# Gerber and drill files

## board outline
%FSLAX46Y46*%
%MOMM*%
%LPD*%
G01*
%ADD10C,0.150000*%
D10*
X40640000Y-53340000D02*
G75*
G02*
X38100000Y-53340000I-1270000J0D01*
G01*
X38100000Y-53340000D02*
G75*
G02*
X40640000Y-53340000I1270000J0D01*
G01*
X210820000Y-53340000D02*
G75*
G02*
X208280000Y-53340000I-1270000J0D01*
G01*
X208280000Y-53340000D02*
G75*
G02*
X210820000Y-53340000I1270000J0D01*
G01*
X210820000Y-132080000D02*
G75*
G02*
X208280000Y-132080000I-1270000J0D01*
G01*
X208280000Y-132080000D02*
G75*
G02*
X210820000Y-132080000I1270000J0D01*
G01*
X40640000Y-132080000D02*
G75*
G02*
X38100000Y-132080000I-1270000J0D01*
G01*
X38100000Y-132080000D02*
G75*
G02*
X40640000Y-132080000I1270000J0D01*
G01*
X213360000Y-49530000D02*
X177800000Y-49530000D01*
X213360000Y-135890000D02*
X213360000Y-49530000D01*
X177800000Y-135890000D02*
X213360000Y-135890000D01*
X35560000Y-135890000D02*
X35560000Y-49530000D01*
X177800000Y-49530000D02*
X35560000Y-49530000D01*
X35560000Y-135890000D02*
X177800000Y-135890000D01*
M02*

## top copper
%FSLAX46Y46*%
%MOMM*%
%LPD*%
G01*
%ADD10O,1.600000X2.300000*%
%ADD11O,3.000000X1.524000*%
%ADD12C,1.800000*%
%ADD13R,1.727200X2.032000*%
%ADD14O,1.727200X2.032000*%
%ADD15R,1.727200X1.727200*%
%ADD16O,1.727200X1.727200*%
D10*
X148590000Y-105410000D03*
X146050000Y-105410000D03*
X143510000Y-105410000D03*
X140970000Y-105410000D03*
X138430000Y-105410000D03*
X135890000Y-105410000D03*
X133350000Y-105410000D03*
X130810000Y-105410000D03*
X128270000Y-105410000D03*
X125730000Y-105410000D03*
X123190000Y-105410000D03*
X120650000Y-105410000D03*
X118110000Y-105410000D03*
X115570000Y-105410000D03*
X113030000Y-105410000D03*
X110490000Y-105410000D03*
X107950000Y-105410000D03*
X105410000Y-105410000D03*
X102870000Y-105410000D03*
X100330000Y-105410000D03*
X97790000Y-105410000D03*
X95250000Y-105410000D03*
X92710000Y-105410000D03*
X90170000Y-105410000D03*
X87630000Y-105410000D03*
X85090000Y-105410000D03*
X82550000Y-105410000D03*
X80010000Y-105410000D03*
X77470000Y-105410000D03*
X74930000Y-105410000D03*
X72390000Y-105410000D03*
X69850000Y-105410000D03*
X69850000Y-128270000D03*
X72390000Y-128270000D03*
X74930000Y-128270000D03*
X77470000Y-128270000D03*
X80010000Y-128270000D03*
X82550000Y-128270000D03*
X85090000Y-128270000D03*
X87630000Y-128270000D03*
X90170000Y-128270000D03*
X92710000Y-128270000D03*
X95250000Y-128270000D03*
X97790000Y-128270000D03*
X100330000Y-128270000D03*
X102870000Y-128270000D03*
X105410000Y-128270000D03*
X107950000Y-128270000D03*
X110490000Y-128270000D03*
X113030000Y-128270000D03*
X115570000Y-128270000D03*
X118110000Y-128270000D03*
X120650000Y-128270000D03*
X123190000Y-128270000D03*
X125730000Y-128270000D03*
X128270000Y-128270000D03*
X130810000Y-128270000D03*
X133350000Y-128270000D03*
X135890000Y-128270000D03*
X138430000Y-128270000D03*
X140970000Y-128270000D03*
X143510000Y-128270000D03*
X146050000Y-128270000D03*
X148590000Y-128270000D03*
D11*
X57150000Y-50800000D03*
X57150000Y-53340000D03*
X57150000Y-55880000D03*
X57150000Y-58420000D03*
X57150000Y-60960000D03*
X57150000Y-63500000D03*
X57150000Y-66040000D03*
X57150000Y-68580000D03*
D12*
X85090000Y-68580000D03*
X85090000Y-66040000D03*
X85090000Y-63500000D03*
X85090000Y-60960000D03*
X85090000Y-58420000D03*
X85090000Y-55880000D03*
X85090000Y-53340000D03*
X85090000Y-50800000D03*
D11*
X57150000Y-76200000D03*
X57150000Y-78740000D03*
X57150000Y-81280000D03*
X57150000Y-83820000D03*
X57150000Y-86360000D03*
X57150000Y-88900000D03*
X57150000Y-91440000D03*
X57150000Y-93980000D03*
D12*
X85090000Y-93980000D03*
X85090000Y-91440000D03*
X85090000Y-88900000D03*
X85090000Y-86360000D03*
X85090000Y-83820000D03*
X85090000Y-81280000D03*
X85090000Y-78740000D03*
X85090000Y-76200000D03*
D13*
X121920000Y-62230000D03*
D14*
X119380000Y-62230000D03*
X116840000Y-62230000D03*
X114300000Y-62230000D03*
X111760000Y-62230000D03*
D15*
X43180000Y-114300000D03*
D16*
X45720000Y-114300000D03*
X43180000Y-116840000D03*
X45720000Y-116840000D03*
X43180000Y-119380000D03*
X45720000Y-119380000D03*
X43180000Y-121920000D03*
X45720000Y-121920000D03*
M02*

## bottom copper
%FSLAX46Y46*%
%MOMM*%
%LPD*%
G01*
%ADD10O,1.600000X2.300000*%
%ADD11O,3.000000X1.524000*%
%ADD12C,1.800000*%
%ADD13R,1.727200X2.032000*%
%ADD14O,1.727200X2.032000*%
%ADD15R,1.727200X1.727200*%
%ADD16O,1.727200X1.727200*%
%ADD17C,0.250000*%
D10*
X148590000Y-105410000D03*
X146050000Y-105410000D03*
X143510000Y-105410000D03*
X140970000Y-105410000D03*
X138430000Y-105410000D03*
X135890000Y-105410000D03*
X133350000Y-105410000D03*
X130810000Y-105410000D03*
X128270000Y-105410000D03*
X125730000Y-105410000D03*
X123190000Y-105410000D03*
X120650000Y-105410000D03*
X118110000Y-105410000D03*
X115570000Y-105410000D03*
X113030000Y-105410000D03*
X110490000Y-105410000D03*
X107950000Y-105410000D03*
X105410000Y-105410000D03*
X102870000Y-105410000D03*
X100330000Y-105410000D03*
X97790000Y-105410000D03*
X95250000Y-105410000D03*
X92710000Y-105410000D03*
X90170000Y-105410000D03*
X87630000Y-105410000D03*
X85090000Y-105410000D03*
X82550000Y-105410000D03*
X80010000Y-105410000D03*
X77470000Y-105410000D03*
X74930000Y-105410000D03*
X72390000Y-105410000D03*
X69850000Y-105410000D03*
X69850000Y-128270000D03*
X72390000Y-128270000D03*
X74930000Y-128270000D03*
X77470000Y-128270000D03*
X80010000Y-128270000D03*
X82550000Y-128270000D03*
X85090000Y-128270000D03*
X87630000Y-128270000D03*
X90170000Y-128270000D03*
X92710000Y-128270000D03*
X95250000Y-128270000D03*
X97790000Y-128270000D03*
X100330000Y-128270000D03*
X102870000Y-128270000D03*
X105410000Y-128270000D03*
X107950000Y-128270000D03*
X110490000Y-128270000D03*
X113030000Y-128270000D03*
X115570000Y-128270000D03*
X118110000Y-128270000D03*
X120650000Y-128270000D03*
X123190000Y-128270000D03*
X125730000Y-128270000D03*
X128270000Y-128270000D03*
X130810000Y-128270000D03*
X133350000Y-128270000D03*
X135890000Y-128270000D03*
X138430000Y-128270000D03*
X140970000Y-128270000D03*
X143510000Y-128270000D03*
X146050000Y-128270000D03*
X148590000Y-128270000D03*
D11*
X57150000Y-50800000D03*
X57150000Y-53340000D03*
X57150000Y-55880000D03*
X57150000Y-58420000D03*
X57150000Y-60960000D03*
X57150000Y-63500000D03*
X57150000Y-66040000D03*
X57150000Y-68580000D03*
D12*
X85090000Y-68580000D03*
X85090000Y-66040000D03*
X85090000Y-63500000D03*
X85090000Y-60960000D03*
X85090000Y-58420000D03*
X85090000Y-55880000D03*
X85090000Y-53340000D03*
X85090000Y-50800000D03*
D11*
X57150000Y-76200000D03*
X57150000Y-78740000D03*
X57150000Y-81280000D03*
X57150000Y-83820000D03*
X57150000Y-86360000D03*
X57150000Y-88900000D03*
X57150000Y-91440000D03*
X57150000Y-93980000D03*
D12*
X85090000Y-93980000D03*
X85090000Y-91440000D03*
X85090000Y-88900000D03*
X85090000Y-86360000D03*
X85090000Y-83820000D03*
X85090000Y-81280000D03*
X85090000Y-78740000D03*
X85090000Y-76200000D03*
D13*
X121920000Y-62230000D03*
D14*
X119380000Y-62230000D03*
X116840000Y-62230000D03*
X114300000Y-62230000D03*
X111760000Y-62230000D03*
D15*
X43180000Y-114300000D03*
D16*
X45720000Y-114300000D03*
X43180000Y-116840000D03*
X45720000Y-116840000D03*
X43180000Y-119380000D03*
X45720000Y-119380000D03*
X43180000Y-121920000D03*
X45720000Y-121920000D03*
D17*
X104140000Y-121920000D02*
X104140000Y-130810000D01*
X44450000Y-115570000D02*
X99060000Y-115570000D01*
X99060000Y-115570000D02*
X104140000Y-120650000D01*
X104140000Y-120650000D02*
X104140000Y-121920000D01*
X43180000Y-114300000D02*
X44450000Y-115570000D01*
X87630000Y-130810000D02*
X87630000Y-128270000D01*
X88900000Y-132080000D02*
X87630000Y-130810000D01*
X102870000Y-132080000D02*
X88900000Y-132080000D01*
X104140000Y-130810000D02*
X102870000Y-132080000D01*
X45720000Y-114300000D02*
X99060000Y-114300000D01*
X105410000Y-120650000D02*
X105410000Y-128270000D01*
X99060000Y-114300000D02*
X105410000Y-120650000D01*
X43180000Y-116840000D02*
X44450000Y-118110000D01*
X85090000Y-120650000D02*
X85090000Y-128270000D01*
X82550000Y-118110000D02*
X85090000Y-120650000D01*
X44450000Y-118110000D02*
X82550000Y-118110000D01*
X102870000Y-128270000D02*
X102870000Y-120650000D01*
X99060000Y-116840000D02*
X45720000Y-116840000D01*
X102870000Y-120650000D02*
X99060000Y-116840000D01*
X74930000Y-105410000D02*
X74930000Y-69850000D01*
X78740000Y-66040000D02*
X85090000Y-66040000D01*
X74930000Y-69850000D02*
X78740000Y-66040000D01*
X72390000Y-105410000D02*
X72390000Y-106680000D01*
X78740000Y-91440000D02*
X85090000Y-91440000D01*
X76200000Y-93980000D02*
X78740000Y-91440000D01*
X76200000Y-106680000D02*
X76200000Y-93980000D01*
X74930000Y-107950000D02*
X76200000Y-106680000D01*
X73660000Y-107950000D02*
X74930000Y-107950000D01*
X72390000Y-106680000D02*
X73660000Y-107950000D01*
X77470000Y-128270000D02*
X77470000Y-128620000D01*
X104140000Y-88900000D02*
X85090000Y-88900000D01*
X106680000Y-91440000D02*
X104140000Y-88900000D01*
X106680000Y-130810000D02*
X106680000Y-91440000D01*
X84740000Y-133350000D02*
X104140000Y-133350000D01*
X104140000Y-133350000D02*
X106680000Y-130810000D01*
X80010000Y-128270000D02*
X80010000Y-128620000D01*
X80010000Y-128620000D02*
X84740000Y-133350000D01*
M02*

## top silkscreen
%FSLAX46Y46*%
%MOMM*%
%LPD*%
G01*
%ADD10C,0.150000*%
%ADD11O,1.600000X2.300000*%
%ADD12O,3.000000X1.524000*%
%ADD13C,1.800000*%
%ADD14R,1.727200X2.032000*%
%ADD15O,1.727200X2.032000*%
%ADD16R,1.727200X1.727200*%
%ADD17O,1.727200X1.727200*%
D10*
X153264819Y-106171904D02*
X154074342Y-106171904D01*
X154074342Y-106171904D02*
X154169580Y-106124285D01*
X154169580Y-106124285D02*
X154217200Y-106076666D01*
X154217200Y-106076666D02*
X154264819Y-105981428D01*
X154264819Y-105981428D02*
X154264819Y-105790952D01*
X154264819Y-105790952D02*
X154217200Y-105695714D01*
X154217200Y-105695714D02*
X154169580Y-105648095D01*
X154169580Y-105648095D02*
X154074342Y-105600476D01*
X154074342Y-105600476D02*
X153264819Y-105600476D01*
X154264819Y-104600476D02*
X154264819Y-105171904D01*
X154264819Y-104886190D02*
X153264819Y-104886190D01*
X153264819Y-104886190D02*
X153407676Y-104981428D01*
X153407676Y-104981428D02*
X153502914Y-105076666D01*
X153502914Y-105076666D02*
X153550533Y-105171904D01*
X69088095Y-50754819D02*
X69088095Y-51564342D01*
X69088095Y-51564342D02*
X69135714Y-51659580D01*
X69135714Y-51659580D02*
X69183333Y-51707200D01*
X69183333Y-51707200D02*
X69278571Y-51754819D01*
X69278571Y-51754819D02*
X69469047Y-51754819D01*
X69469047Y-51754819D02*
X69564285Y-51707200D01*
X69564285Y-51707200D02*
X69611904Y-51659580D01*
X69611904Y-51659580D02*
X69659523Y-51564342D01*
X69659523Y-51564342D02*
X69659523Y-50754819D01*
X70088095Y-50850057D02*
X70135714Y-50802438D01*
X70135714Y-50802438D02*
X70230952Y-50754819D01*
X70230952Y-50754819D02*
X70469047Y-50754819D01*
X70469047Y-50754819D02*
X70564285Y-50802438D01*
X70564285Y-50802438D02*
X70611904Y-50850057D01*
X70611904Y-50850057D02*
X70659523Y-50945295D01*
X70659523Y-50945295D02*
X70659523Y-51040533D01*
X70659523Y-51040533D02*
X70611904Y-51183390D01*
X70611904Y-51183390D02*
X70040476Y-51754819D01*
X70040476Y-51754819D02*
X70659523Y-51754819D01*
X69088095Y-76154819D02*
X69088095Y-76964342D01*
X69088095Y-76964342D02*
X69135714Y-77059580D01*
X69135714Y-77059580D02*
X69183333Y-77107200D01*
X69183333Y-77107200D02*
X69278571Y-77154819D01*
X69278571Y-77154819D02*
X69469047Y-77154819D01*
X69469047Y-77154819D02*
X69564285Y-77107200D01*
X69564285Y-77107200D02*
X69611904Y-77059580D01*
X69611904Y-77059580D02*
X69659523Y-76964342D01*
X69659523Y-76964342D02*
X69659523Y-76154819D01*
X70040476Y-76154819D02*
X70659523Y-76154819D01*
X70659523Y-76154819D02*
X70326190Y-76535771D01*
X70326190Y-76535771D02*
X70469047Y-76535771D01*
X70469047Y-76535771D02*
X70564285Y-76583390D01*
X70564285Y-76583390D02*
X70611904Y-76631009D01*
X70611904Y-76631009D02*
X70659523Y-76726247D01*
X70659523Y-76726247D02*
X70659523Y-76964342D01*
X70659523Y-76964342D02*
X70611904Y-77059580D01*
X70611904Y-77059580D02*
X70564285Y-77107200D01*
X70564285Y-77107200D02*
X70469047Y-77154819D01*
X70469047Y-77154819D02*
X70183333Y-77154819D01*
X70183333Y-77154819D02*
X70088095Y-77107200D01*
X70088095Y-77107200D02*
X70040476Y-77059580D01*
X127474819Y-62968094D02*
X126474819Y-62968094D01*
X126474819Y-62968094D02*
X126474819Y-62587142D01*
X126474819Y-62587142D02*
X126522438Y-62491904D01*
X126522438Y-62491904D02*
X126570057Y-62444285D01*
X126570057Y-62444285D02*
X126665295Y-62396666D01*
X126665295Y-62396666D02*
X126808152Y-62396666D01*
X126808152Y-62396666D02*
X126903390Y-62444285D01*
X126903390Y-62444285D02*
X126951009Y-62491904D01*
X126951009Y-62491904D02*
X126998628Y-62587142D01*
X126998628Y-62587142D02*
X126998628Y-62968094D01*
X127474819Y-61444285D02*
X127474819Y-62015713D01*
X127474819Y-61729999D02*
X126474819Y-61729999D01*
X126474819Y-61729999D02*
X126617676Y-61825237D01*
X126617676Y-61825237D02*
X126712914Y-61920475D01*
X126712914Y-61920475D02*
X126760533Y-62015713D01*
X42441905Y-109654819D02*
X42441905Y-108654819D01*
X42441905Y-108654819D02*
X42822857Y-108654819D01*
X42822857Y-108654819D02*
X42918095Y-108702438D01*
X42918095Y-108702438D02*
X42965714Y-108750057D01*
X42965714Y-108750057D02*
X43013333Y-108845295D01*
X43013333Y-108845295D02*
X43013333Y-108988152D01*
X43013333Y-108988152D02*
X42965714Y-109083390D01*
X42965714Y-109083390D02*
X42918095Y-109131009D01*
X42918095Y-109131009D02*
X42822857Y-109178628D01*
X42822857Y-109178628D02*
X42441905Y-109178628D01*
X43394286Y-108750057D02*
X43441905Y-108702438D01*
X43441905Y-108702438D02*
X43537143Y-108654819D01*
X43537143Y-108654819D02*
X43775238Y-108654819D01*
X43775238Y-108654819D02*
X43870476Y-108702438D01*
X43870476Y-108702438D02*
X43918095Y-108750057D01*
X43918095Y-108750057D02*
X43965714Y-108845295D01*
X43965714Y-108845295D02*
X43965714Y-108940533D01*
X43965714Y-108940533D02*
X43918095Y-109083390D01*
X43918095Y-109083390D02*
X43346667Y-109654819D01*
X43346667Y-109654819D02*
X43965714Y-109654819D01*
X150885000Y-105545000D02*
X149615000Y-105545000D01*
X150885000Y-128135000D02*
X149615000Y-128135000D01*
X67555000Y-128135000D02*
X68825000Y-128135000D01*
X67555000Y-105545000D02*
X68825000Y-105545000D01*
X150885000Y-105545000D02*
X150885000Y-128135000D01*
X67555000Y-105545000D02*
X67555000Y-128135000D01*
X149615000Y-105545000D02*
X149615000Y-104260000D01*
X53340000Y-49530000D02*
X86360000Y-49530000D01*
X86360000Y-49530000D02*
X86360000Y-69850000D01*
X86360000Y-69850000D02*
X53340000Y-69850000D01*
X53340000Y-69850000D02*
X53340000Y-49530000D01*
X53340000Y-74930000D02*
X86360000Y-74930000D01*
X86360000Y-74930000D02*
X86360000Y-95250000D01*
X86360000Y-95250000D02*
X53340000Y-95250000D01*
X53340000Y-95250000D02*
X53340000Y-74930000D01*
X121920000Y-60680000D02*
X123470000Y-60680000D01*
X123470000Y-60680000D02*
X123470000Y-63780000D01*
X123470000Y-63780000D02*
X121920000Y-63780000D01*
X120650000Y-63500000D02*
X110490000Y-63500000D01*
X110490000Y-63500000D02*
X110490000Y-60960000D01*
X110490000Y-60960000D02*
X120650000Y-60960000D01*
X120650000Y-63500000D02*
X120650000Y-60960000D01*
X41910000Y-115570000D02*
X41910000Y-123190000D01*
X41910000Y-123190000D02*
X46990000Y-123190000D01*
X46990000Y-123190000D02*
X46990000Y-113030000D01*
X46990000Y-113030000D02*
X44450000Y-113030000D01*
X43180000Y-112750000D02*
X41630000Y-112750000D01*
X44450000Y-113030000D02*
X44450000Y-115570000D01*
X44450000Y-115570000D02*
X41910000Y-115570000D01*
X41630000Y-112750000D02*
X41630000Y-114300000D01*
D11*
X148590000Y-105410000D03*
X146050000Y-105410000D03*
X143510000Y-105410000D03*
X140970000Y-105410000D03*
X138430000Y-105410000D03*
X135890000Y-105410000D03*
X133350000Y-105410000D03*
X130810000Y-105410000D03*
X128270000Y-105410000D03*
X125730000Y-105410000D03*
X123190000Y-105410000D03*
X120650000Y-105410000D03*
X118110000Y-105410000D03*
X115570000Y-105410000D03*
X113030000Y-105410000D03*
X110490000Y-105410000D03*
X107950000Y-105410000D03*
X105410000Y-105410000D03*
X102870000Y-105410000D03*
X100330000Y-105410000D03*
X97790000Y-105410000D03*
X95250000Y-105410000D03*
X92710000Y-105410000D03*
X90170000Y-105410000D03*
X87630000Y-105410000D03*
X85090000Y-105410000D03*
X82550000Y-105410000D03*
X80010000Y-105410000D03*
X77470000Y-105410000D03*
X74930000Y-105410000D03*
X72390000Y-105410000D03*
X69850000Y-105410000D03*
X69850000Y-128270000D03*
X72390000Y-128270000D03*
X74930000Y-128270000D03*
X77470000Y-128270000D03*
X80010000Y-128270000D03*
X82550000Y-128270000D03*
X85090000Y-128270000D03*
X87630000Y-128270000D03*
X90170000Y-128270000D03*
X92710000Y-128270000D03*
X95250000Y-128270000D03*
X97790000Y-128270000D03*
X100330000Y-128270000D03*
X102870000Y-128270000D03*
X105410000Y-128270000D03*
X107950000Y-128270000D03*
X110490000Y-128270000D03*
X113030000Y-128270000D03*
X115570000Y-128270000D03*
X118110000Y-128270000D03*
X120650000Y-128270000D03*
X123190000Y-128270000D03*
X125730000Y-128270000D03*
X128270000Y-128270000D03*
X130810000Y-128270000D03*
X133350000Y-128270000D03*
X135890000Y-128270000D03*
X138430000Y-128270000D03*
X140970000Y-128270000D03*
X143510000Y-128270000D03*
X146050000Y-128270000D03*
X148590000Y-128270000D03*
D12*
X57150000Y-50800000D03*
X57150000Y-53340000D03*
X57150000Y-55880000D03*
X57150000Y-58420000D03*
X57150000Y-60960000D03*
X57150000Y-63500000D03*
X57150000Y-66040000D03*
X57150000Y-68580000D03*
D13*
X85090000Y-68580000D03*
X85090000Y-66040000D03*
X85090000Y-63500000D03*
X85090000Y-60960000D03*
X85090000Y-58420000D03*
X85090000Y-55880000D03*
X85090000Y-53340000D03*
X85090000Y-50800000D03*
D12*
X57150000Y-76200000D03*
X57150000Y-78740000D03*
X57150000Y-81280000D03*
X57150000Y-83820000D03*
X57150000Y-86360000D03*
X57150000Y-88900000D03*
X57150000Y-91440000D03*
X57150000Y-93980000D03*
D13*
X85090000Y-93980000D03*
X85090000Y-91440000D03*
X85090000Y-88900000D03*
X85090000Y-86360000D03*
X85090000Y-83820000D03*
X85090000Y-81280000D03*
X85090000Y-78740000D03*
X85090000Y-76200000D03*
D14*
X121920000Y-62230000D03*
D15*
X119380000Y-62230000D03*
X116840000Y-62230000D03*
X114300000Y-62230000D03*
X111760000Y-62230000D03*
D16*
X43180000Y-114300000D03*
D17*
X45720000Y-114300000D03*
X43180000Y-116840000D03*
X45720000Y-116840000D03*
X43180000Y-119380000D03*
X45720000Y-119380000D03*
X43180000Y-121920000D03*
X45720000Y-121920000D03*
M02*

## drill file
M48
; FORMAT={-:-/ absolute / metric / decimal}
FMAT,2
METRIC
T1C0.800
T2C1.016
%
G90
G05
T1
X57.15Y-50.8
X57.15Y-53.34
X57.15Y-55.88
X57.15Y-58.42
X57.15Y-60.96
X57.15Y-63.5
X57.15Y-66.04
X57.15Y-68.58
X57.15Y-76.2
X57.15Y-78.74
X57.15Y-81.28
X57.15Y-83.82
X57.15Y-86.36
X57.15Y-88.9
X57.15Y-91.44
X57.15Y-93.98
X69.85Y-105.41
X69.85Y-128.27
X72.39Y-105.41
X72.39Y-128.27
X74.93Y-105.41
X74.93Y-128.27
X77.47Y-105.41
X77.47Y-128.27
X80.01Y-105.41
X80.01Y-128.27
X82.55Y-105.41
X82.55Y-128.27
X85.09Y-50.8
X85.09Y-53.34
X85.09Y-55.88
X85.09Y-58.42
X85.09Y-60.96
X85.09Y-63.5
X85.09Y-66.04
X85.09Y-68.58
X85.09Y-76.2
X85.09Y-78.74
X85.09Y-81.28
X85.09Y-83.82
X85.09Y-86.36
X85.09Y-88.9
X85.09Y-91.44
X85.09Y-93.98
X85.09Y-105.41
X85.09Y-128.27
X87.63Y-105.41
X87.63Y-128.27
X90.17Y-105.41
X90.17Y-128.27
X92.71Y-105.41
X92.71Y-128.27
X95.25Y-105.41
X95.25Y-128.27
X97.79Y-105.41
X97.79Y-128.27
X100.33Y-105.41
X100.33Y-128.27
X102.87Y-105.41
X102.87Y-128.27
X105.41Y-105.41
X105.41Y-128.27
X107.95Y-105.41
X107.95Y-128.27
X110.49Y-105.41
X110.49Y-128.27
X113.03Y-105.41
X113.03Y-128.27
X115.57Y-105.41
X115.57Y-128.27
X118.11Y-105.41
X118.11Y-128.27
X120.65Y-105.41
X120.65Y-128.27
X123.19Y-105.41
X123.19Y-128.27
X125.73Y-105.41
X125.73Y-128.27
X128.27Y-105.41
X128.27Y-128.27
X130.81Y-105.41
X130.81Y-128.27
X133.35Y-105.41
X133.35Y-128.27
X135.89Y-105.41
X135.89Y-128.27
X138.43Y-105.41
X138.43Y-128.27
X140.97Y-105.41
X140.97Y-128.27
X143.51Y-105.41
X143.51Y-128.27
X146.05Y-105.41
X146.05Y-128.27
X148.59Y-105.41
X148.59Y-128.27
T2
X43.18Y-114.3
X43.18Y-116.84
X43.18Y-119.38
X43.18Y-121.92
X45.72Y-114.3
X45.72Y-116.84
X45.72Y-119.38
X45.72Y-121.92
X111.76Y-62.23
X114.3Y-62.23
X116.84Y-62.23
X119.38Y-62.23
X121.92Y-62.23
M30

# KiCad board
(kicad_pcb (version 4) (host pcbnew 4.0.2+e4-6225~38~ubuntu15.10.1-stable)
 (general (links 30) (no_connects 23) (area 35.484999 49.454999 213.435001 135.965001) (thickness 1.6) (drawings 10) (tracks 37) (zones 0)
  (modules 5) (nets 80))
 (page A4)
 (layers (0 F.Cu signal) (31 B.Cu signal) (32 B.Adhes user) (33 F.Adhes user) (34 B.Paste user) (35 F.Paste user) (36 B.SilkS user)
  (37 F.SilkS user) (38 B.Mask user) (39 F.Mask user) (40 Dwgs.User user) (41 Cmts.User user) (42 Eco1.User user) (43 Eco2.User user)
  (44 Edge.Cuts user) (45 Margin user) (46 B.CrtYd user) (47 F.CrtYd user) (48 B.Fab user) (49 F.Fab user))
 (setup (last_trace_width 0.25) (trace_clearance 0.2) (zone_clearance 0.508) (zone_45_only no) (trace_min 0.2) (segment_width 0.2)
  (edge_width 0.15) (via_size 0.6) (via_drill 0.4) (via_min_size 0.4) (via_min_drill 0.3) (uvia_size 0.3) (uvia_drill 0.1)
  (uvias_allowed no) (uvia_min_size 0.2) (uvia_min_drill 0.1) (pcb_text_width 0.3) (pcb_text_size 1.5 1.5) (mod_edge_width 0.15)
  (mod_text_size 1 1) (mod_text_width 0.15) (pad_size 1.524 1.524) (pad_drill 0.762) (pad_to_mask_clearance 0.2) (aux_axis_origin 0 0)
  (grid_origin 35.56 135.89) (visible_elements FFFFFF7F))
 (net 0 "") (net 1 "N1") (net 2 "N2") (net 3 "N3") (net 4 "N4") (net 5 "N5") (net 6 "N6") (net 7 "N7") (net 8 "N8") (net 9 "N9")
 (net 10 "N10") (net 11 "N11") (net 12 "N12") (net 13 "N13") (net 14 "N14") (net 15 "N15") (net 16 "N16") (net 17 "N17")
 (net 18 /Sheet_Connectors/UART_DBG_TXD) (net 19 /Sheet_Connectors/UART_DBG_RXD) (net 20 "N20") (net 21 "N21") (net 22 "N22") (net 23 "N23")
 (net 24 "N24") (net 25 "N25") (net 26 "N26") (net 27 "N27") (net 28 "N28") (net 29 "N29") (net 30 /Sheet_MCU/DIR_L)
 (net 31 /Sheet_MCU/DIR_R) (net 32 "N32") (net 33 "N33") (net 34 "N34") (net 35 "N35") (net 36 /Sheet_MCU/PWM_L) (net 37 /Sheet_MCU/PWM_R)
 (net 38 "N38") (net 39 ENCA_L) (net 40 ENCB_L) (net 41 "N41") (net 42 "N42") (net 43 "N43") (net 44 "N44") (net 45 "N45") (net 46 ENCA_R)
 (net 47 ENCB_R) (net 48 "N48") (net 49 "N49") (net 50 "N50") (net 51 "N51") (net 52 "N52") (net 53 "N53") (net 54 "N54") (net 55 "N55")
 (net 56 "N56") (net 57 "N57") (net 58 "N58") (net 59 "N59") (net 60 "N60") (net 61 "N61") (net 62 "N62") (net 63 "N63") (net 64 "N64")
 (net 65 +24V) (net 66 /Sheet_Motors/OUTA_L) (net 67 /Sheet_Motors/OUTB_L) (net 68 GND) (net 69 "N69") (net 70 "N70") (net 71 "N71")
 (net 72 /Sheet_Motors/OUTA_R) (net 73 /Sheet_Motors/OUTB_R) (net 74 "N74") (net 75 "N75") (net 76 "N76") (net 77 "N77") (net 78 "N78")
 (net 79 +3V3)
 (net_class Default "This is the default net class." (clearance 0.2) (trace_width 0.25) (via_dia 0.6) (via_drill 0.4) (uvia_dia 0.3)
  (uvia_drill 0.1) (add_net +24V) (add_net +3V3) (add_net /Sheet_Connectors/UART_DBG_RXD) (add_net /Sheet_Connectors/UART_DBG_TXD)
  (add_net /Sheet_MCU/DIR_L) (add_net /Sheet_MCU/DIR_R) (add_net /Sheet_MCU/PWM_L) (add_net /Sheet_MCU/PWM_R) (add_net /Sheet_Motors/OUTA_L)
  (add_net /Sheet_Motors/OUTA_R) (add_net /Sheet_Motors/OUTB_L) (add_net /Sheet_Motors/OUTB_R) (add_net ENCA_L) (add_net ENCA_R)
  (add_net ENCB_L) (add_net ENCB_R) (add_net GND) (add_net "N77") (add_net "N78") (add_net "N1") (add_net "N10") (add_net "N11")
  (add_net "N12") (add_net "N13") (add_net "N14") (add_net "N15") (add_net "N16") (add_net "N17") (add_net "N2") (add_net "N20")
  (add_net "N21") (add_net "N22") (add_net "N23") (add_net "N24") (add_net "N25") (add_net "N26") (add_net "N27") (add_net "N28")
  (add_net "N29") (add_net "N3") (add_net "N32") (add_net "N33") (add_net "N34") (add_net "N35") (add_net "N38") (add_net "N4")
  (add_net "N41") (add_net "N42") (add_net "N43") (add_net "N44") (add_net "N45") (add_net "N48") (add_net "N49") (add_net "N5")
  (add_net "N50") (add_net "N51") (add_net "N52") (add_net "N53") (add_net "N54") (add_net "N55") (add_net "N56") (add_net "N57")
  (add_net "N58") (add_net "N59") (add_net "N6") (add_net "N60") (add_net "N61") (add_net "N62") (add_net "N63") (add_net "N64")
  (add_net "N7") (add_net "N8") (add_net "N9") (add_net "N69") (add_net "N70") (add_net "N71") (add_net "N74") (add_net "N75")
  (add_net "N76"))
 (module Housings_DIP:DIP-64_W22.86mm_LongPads (layer F.Cu) (at 148.59 105.41 270)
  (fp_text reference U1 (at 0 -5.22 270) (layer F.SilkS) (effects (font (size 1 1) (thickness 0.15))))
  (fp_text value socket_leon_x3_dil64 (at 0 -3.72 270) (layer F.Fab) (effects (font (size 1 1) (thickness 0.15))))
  (fp_line (start 0.135 -2.295) (end 0.135 -1.025) (layer F.SilkS) (width 0.15))
  (fp_line (start 22.725 -2.295) (end 22.725 -1.025) (layer F.SilkS) (width 0.15))
  (fp_line (start 22.725 81.035) (end 22.725 79.765) (layer F.SilkS) (width 0.15))
  (fp_line (start 0.135 81.035) (end 0.135 79.765) (layer F.SilkS) (width 0.15))
  (fp_line (start 0.135 -2.295) (end 22.725 -2.295) (layer F.SilkS) (width 0.15))
  (fp_line (start 0.135 81.035) (end 22.725 81.035) (layer F.SilkS) (width 0.15))
  (fp_line (start 0.135 -1.025) (end -1.15 -1.025) (layer F.SilkS) (width 0.15))
  (pad 1 thru_hole oval (at 0 0 270) (size 2.3 1.6) (drill 0.8) (layers *.Cu *.Mask F.SilkS) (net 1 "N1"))
  (pad 2 thru_hole oval (at 0 2.54 270) (size 2.3 1.6) (drill 0.8) (layers *.Cu *.Mask F.SilkS) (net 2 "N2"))
  (pad 3 thru_hole oval (at 0 5.08 270) (size 2.3 1.6) (drill 0.8) (layers *.Cu *.Mask F.SilkS) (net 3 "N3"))
  (pad 4 thru_hole oval (at 0 7.62 270) (size 2.3 1.6) (drill 0.8) (layers *.Cu *.Mask F.SilkS) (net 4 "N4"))
  (pad 5 thru_hole oval (at 0 10.16 270) (size 2.3 1.6) (drill 0.8) (layers *.Cu *.Mask F.SilkS) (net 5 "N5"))
  (pad 6 thru_hole oval (at 0 12.7 270) (size 2.3 1.6) (drill 0.8) (layers *.Cu *.Mask F.SilkS) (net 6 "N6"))
  (pad 7 thru_hole oval (at 0 15.24 270) (size 2.3 1.6) (drill 0.8) (layers *.Cu *.Mask F.SilkS) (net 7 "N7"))
  (pad 8 thru_hole oval (at 0 17.78 270) (size 2.3 1.6) (drill 0.8) (layers *.Cu *.Mask F.SilkS) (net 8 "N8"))
  (pad 9 thru_hole oval (at 0 20.32 270) (size 2.3 1.6) (drill 0.8) (layers *.Cu *.Mask F.SilkS) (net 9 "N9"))
  (pad 10 thru_hole oval (at 0 22.86 270) (size 2.3 1.6) (drill 0.8) (layers *.Cu *.Mask F.SilkS) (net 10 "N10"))
  (pad 11 thru_hole oval (at 0 25.4 270) (size 2.3 1.6) (drill 0.8) (layers *.Cu *.Mask F.SilkS) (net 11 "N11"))
  (pad 12 thru_hole oval (at 0 27.94 270) (size 2.3 1.6) (drill 0.8) (layers *.Cu *.Mask F.SilkS) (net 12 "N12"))
  (pad 13 thru_hole oval (at 0 30.48 270) (size 2.3 1.6) (drill 0.8) (layers *.Cu *.Mask F.SilkS) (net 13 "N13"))
  (pad 14 thru_hole oval (at 0 33.02 270) (size 2.3 1.6) (drill 0.8) (layers *.Cu *.Mask F.SilkS) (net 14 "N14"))
  (pad 15 thru_hole oval (at 0 35.56 270) (size 2.3 1.6) (drill 0.8) (layers *.Cu *.Mask F.SilkS) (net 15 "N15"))
  (pad 16 thru_hole oval (at 0 38.1 270) (size 2.3 1.6) (drill 0.8) (layers *.Cu *.Mask F.SilkS) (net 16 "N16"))
  (pad 17 thru_hole oval (at 0 40.64 270) (size 2.3 1.6) (drill 0.8) (layers *.Cu *.Mask F.SilkS) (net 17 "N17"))
  (pad 18 thru_hole oval (at 0 43.18 270) (size 2.3 1.6) (drill 0.8) (layers *.Cu *.Mask F.SilkS) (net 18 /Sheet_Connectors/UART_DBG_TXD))
  (pad 19 thru_hole oval (at 0 45.72 270) (size 2.3 1.6) (drill 0.8) (layers *.Cu *.Mask F.SilkS) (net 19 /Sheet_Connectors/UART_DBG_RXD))
  (pad 20 thru_hole oval (at 0 48.26 270) (size 2.3 1.6) (drill 0.8) (layers *.Cu *.Mask F.SilkS) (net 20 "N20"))
  (pad 21 thru_hole oval (at 0 50.8 270) (size 2.3 1.6) (drill 0.8) (layers *.Cu *.Mask F.SilkS) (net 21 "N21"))
  (pad 22 thru_hole oval (at 0 53.34 270) (size 2.3 1.6) (drill 0.8) (layers *.Cu *.Mask F.SilkS) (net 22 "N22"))
  (pad 23 thru_hole oval (at 0 55.88 270) (size 2.3 1.6) (drill 0.8) (layers *.Cu *.Mask F.SilkS) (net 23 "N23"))
  (pad 24 thru_hole oval (at 0 58.42 270) (size 2.3 1.6) (drill 0.8) (layers *.Cu *.Mask F.SilkS) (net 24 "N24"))
  (pad 25 thru_hole oval (at 0 60.96 270) (size 2.3 1.6) (drill 0.8) (layers *.Cu *.Mask F.SilkS) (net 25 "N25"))
  (pad 26 thru_hole oval (at 0 63.5 270) (size 2.3 1.6) (drill 0.8) (layers *.Cu *.Mask F.SilkS) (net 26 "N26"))
  (pad 27 thru_hole oval (at 0 66.04 270) (size 2.3 1.6) (drill 0.8) (layers *.Cu *.Mask F.SilkS) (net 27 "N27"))
  (pad 28 thru_hole oval (at 0 68.58 270) (size 2.3 1.6) (drill 0.8) (layers *.Cu *.Mask F.SilkS) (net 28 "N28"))
  (pad 29 thru_hole oval (at 0 71.12 270) (size 2.3 1.6) (drill 0.8) (layers *.Cu *.Mask F.SilkS) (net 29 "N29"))
  (pad 30 thru_hole oval (at 0 73.66 270) (size 2.3 1.6) (drill 0.8) (layers *.Cu *.Mask F.SilkS) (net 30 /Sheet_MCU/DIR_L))
  (pad 31 thru_hole oval (at 0 76.2 270) (size 2.3 1.6) (drill 0.8) (layers *.Cu *.Mask F.SilkS) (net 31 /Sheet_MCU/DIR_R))
  (pad 32 thru_hole oval (at 0 78.74 270) (size 2.3 1.6) (drill 0.8) (layers *.Cu *.Mask F.SilkS) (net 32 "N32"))
  (pad 33 thru_hole oval (at 22.86 78.74 270) (size 2.3 1.6) (drill 0.8) (layers *.Cu *.Mask F.SilkS) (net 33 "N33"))
  (pad 34 thru_hole oval (at 22.86 76.2 270) (size 2.3 1.6) (drill 0.8) (layers *.Cu *.Mask F.SilkS) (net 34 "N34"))
  (pad 35 thru_hole oval (at 22.86 73.66 270) (size 2.3 1.6) (drill 0.8) (layers *.Cu *.Mask F.SilkS) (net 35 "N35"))
  (pad 36 thru_hole oval (at 22.86 71.12 270) (size 2.3 1.6) (drill 0.8) (layers *.Cu *.Mask F.SilkS) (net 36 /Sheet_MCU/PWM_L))
  (pad 37 thru_hole oval (at 22.86 68.58 270) (size 2.3 1.6) (drill 0.8) (layers *.Cu *.Mask F.SilkS) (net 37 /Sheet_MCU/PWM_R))
  (pad 38 thru_hole oval (at 22.86 66.04 270) (size 2.3 1.6) (drill 0.8) (layers *.Cu *.Mask F.SilkS) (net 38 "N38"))
  (pad 39 thru_hole oval (at 22.86 63.5 270) (size 2.3 1.6) (drill 0.8) (layers *.Cu *.Mask F.SilkS) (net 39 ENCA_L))
  (pad 40 thru_hole oval (at 22.86 60.96 270) (size 2.3 1.6) (drill 0.8) (layers *.Cu *.Mask F.SilkS) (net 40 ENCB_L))
  (pad 41 thru_hole oval (at 22.86 58.42 270) (size 2.3 1.6) (drill 0.8) (layers *.Cu *.Mask F.SilkS) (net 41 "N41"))
  (pad 42 thru_hole oval (at 22.86 55.88 270) (size 2.3 1.6) (drill 0.8) (layers *.Cu *.Mask F.SilkS) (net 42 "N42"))
  (pad 43 thru_hole oval (at 22.86 53.34 270) (size 2.3 1.6) (drill 0.8) (layers *.Cu *.Mask F.SilkS) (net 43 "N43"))
  (pad 44 thru_hole oval (at 22.86 50.8 270) (size 2.3 1.6) (drill 0.8) (layers *.Cu *.Mask F.SilkS) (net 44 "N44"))
  (pad 45 thru_hole oval (at 22.86 48.26 270) (size 2.3 1.6) (drill 0.8) (layers *.Cu *.Mask F.SilkS) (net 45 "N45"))
  (pad 46 thru_hole oval (at 22.86 45.72 270) (size 2.3 1.6) (drill 0.8) (layers *.Cu *.Mask F.SilkS) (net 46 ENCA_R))
  (pad 47 thru_hole oval (at 22.86 43.18 270) (size 2.3 1.6) (drill 0.8) (layers *.Cu *.Mask F.SilkS) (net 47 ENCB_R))
  (pad 48 thru_hole oval (at 22.86 40.64 270) (size 2.3 1.6) (drill 0.8) (layers *.Cu *.Mask F.SilkS) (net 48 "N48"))
  (pad 49 thru_hole oval (at 22.86 38.1 270) (size 2.3 1.6) (drill 0.8) (layers *.Cu *.Mask F.SilkS) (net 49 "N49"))
  (pad 50 thru_hole oval (at 22.86 35.56 270) (size 2.3 1.6) (drill 0.8) (layers *.Cu *.Mask F.SilkS) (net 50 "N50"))
  (pad 51 thru_hole oval (at 22.86 33.02 270) (size 2.3 1.6) (drill 0.8) (layers *.Cu *.Mask F.SilkS) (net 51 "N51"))
  (pad 52 thru_hole oval (at 22.86 30.48 270) (size 2.3 1.6) (drill 0.8) (layers *.Cu *.Mask F.SilkS) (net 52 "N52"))
  (pad 53 thru_hole oval (at 22.86 27.94 270) (size 2.3 1.6) (drill 0.8) (layers *.Cu *.Mask F.SilkS) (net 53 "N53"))
  (pad 54 thru_hole oval (at 22.86 25.4 270) (size 2.3 1.6) (drill 0.8) (layers *.Cu *.Mask F.SilkS) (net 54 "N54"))
  (pad 55 thru_hole oval (at 22.86 22.86 270) (size 2.3 1.6) (drill 0.8) (layers *.Cu *.Mask F.SilkS) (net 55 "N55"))
  (pad 56 thru_hole oval (at 22.86 20.32 270) (size 2.3 1.6) (drill 0.8) (layers *.Cu *.Mask F.SilkS) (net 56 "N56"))
  (pad 57 thru_hole oval (at 22.86 17.78 270) (size 2.3 1.6) (drill 0.8) (layers *.Cu *.Mask F.SilkS) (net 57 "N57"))
  (pad 58 thru_hole oval (at 22.86 15.24 270) (size 2.3 1.6) (drill 0.8) (layers *.Cu *.Mask F.SilkS) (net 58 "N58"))
  (pad 59 thru_hole oval (at 22.86 12.7 270) (size 2.3 1.6) (drill 0.8) (layers *.Cu *.Mask F.SilkS) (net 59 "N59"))
  (pad 60 thru_hole oval (at 22.86 10.16 270) (size 2.3 1.6) (drill 0.8) (layers *.Cu *.Mask F.SilkS) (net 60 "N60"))
  (pad 61 thru_hole oval (at 22.86 7.62 270) (size 2.3 1.6) (drill 0.8) (layers *.Cu *.Mask F.SilkS) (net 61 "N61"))
  (pad 62 thru_hole oval (at 22.86 5.08 270) (size 2.3 1.6) (drill 0.8) (layers *.Cu *.Mask F.SilkS) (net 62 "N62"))
  (pad 63 thru_hole oval (at 22.86 2.54 270) (size 2.3 1.6) (drill 0.8) (layers *.Cu *.Mask F.SilkS) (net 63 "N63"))
  (pad 64 thru_hole oval (at 22.86 0 270) (size 2.3 1.6) (drill 0.8) (layers *.Cu *.Mask F.SilkS) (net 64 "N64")))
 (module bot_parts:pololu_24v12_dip (layer F.Cu) (at 69.85 59.69)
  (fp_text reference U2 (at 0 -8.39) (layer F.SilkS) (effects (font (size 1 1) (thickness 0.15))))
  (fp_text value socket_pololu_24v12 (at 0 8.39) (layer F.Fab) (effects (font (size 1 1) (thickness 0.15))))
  (fp_line (start -16.51 -10.16) (end 16.51 -10.16) (layer F.SilkS) (width 0.15))
  (fp_line (start 16.51 -10.16) (end 16.51 10.16) (layer F.SilkS) (width 0.15))
  (fp_line (start 16.51 10.16) (end -16.51 10.16) (layer F.SilkS) (width 0.15))
  (fp_line (start -16.51 10.16) (end -16.51 -10.16) (layer F.SilkS) (width 0.15))
  (pad 1 thru_hole oval (at -12.7 -8.89) (size 3 1.524) (drill 0.8) (layers *.Cu *.Mask F.SilkS) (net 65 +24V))
  (pad 2 thru_hole oval (at -12.7 -6.35) (size 3 1.524) (drill 0.8) (layers *.Cu *.Mask F.SilkS) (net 65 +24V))
  (pad 3 thru_hole oval (at -12.7 -3.81) (size 3 1.524) (drill 0.8) (layers *.Cu *.Mask F.SilkS) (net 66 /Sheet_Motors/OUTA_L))
  (pad 4 thru_hole oval (at -12.7 -1.27) (size 3 1.524) (drill 0.8) (layers *.Cu *.Mask F.SilkS) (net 66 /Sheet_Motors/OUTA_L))
  (pad 5 thru_hole oval (at -12.7 1.27) (size 3 1.524) (drill 0.8) (layers *.Cu *.Mask F.SilkS) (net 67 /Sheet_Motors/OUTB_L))
  (pad 6 thru_hole oval (at -12.7 3.81) (size 3 1.524) (drill 0.8) (layers *.Cu *.Mask F.SilkS) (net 67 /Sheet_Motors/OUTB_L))
  (pad 7 thru_hole oval (at -12.7 6.35) (size 3 1.524) (drill 0.8) (layers *.Cu *.Mask F.SilkS) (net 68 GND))
  (pad 8 thru_hole oval (at -12.7 8.89) (size 3 1.524) (drill 0.8) (layers *.Cu *.Mask F.SilkS) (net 68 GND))
  (pad 9 thru_hole circle (at 15.24 8.89) (size 1.8 1.8) (drill 0.8) (layers *.Cu *.Mask F.SilkS) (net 68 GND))
  (pad 10 thru_hole circle (at 15.24 6.35) (size 1.8 1.8) (drill 0.8) (layers *.Cu *.Mask F.SilkS) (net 30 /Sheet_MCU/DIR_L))
  (pad 11 thru_hole circle (at 15.24 3.81) (size 1.8 1.8) (drill 0.8) (layers *.Cu *.Mask F.SilkS) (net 36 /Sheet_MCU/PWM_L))
  (pad 12 thru_hole circle (at 15.24 1.27) (size 1.8 1.8) (drill 0.8) (layers *.Cu *.Mask F.SilkS) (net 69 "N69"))
  (pad 13 thru_hole circle (at 15.24 -1.27) (size 1.8 1.8) (drill 0.8) (layers *.Cu *.Mask F.SilkS) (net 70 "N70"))
  (pad 14 thru_hole circle (at 15.24 -3.81) (size 1.8 1.8) (drill 0.8) (layers *.Cu *.Mask F.SilkS) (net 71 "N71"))
  (pad 15 thru_hole circle (at 15.24 -6.35) (size 1.8 1.8) (drill 0.8) (layers *.Cu *.Mask F.SilkS) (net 65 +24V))
  (pad 16 thru_hole circle (at 15.24 -8.89) (size 1.8 1.8) (drill 0.8) (layers *.Cu *.Mask F.SilkS) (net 65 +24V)))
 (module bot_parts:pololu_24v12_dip (layer F.Cu) (at 69.85 85.09)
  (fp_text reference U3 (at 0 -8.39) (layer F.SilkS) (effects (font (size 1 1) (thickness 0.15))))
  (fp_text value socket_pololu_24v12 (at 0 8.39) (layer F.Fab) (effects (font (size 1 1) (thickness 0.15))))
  (fp_line (start -16.51 -10.16) (end 16.51 -10.16) (layer F.SilkS) (width 0.15))
  (fp_line (start 16.51 -10.16) (end 16.51 10.16) (layer F.SilkS) (width 0.15))
  (fp_line (start 16.51 10.16) (end -16.51 10.16) (layer F.SilkS) (width 0.15))
  (fp_line (start -16.51 10.16) (end -16.51 -10.16) (layer F.SilkS) (width 0.15))
  (pad 1 thru_hole oval (at -12.7 -8.89) (size 3 1.524) (drill 0.8) (layers *.Cu *.Mask F.SilkS) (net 65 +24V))
  (pad 2 thru_hole oval (at -12.7 -6.35) (size 3 1.524) (drill 0.8) (layers *.Cu *.Mask F.SilkS) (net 65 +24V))
  (pad 3 thru_hole oval (at -12.7 -3.81) (size 3 1.524) (drill 0.8) (layers *.Cu *.Mask F.SilkS) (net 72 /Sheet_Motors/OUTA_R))
  (pad 4 thru_hole oval (at -12.7 -1.27) (size 3 1.524) (drill 0.8) (layers *.Cu *.Mask F.SilkS) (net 72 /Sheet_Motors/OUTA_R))
  (pad 5 thru_hole oval (at -12.7 1.27) (size 3 1.524) (drill 0.8) (layers *.Cu *.Mask F.SilkS) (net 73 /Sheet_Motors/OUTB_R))
  (pad 6 thru_hole oval (at -12.7 3.81) (size 3 1.524) (drill 0.8) (layers *.Cu *.Mask F.SilkS) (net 73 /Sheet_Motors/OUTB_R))
  (pad 7 thru_hole oval (at -12.7 6.35) (size 3 1.524) (drill 0.8) (layers *.Cu *.Mask F.SilkS) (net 68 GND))
  (pad 8 thru_hole oval (at -12.7 8.89) (size 3 1.524) (drill 0.8) (layers *.Cu *.Mask F.SilkS) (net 68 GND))
  (pad 9 thru_hole circle (at 15.24 8.89) (size 1.8 1.8) (drill 0.8) (layers *.Cu *.Mask F.SilkS) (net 68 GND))
  (pad 10 thru_hole circle (at 15.24 6.35) (size 1.8 1.8) (drill 0.8) (layers *.Cu *.Mask F.SilkS) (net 31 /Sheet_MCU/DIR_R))
  (pad 11 thru_hole circle (at 15.24 3.81) (size 1.8 1.8) (drill 0.8) (layers *.Cu *.Mask F.SilkS) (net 37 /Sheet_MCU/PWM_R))
  (pad 12 thru_hole circle (at 15.24 1.27) (size 1.8 1.8) (drill 0.8) (layers *.Cu *.Mask F.SilkS) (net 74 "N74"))
  (pad 13 thru_hole circle (at 15.24 -1.27) (size 1.8 1.8) (drill 0.8) (layers *.Cu *.Mask F.SilkS) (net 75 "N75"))
  (pad 14 thru_hole circle (at 15.24 -3.81) (size 1.8 1.8) (drill 0.8) (layers *.Cu *.Mask F.SilkS) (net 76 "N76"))
  (pad 15 thru_hole circle (at 15.24 -6.35) (size 1.8 1.8) (drill 0.8) (layers *.Cu *.Mask F.SilkS) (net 65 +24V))
  (pad 16 thru_hole circle (at 15.24 -8.89) (size 1.8 1.8) (drill 0.8) (layers *.Cu *.Mask F.SilkS) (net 65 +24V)))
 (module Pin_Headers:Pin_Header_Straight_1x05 (layer F.Cu) (at 121.92 62.23 270)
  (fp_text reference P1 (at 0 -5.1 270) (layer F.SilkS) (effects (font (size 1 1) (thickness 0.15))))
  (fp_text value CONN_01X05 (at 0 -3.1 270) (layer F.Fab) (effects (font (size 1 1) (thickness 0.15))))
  (fp_line (start -1.55 0) (end -1.55 -1.55) (layer F.SilkS) (width 0.15))
  (fp_line (start -1.55 -1.55) (end 1.55 -1.55) (layer F.SilkS) (width 0.15))
  (fp_line (start 1.55 -1.55) (end 1.55 0) (layer F.SilkS) (width 0.15))
  (fp_line (start 1.27 1.27) (end 1.27 11.43) (layer F.SilkS) (width 0.15))
  (fp_line (start 1.27 11.43) (end -1.27 11.43) (layer F.SilkS) (width 0.15))
  (fp_line (start -1.27 11.43) (end -1.27 1.27) (layer F.SilkS) (width 0.15))
  (fp_line (start 1.27 1.27) (end -1.27 1.27) (layer F.SilkS) (width 0.15))
  (pad 1 thru_hole rect (at 0 0 270) (size 2.032 1.7272) (drill 1.016) (layers *.Cu *.Mask F.SilkS) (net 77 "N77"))
  (pad 2 thru_hole oval (at 0 2.54 270) (size 2.032 1.7272) (drill 1.016) (layers *.Cu *.Mask F.SilkS)
   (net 18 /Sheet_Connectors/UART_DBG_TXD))
  (pad 3 thru_hole oval (at 0 5.08 270) (size 2.032 1.7272) (drill 1.016) (layers *.Cu *.Mask F.SilkS)
   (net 19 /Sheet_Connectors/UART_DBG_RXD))
  (pad 4 thru_hole oval (at 0 7.62 270) (size 2.032 1.7272) (drill 1.016) (layers *.Cu *.Mask F.SilkS) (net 68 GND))
  (pad 5 thru_hole oval (at 0 10.16 270) (size 2.032 1.7272) (drill 1.016) (layers *.Cu *.Mask F.SilkS) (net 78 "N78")))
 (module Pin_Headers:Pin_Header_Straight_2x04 (layer F.Cu) (at 43.18 114.3)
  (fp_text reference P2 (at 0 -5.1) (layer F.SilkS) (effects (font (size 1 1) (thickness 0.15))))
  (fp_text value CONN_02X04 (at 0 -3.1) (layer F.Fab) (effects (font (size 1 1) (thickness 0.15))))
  (fp_line (start -1.27 1.27) (end -1.27 8.89) (layer F.SilkS) (width 0.15))
  (fp_line (start -1.27 8.89) (end 3.81 8.89) (layer F.SilkS) (width 0.15))
  (fp_line (start 3.81 8.89) (end 3.81 -1.27) (layer F.SilkS) (width 0.15))
  (fp_line (start 3.81 -1.27) (end 1.27 -1.27) (layer F.SilkS) (width 0.15))
  (fp_line (start 0 -1.55) (end -1.55 -1.55) (layer F.SilkS) (width 0.15))
  (fp_line (start 1.27 -1.27) (end 1.27 1.27) (layer F.SilkS) (width 0.15))
  (fp_line (start 1.27 1.27) (end -1.27 1.27) (layer F.SilkS) (width 0.15))
  (fp_line (start -1.55 -1.55) (end -1.55 0) (layer F.SilkS) (width 0.15))
  (pad 1 thru_hole rect (at 0 0) (size 1.7272 1.7272) (drill 1.016) (layers *.Cu *.Mask F.SilkS) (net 40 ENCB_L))
  (pad 2 thru_hole oval (at 2.54 0) (size 1.7272 1.7272) (drill 1.016) (layers *.Cu *.Mask F.SilkS) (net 47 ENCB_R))
  (pad 3 thru_hole oval (at 0 2.54) (size 1.7272 1.7272) (drill 1.016) (layers *.Cu *.Mask F.SilkS) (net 39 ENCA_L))
  (pad 4 thru_hole oval (at 2.54 2.54) (size 1.7272 1.7272) (drill 1.016) (layers *.Cu *.Mask F.SilkS) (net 46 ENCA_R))
  (pad 5 thru_hole oval (at 0 5.08) (size 1.7272 1.7272) (drill 1.016) (layers *.Cu *.Mask F.SilkS) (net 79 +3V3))
  (pad 6 thru_hole oval (at 2.54 5.08) (size 1.7272 1.7272) (drill 1.016) (layers *.Cu *.Mask F.SilkS) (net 79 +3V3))
  (pad 7 thru_hole oval (at 0 7.62) (size 1.7272 1.7272) (drill 1.016) (layers *.Cu *.Mask F.SilkS) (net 68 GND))
  (pad 8 thru_hole oval (at 2.54 7.62) (size 1.7272 1.7272) (drill 1.016) (layers *.Cu *.Mask F.SilkS) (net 68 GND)))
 (gr_circle (center 39.37 53.34) (end 40.64 53.34) (layer Edge.Cuts) (width 0.15))
 (gr_circle (center 209.55 53.34) (end 209.55 52.07) (layer Edge.Cuts) (width 0.15))
 (gr_circle (center 209.55 132.08) (end 210.82 132.08) (layer Edge.Cuts) (width 0.15))
 (gr_circle (center 39.37 132.08) (end 40.64 132.08) (layer Edge.Cuts) (width 0.15))
 (gr_line (start 213.36 49.53) (end 177.8 49.53) (angle 90) (layer Edge.Cuts) (width 0.15))
 (gr_line (start 213.36 135.89) (end 213.36 49.53) (angle 90) (layer Edge.Cuts) (width 0.15))
 (gr_line (start 177.8 135.89) (end 213.36 135.89) (angle 90) (layer Edge.Cuts) (width 0.15))
 (gr_line (start 35.56 135.89) (end 35.56 49.53) (angle 90) (layer Edge.Cuts) (width 0.15))
 (gr_line (start 177.8 49.53) (end 35.56 49.53) (angle 90) (layer Edge.Cuts) (width 0.15))
 (gr_line (start 35.56 135.89) (end 177.8 135.89) (angle 90) (layer Edge.Cuts) (width 0.15))
 (segment (start 104.14 121.92) (end 104.14 130.81) (width 0.25) (layer B.Cu) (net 40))
 (segment (start 44.45 115.57) (end 99.06 115.57) (width 0.25) (layer B.Cu) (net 40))
 (segment (start 99.06 115.57) (end 104.14 120.65) (width 0.25) (layer B.Cu) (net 40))
 (segment (start 104.14 120.65) (end 104.14 121.92) (width 0.25) (layer B.Cu) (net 40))
 (segment (start 43.18 114.3) (end 44.45 115.57) (width 0.25) (layer B.Cu) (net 40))
 (segment (start 87.63 130.81) (end 87.63 128.27) (width 0.25) (layer B.Cu) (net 40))
 (segment (start 88.9 132.08) (end 87.63 130.81) (width 0.25) (layer B.Cu) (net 40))
 (segment (start 102.87 132.08) (end 88.9 132.08) (width 0.25) (layer B.Cu) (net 40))
 (segment (start 104.14 130.81) (end 102.87 132.08) (width 0.25) (layer B.Cu) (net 40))
 (segment (start 45.72 114.3) (end 99.06 114.3) (width 0.25) (layer B.Cu) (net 47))
 (segment (start 105.41 120.65) (end 105.41 128.27) (width 0.25) (layer B.Cu) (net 47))
 (segment (start 99.06 114.3) (end 105.41 120.65) (width 0.25) (layer B.Cu) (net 47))
 (segment (start 43.18 116.84) (end 44.45 118.11) (width 0.25) (layer B.Cu) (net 39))
 (segment (start 85.09 120.65) (end 85.09 128.27) (width 0.25) (layer B.Cu) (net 39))
 (segment (start 82.55 118.11) (end 85.09 120.65) (width 0.25) (layer B.Cu) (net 39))
 (segment (start 44.45 118.11) (end 82.55 118.11) (width 0.25) (layer B.Cu) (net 39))
 (segment (start 102.87 128.27) (end 102.87 120.65) (width 0.25) (layer B.Cu) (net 46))
 (segment (start 99.06 116.84) (end 45.72 116.84) (width 0.25) (layer B.Cu) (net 46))
 (segment (start 102.87 120.65) (end 99.06 116.84) (width 0.25) (layer B.Cu) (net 46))
 (segment (start 74.93 105.41) (end 74.93 69.85) (width 0.25) (layer B.Cu) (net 30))
 (segment (start 78.74 66.04) (end 85.09 66.04) (width 0.25) (layer B.Cu) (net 30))
 (segment (start 74.93 69.85) (end 78.74 66.04) (width 0.25) (layer B.Cu) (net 30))
 (segment (start 72.39 105.41) (end 72.39 106.68) (width 0.25) (layer B.Cu) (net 31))
 (segment (start 78.74 91.44) (end 85.09 91.44) (width 0.25) (layer B.Cu) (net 31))
 (segment (start 76.2 93.98) (end 78.74 91.44) (width 0.25) (layer B.Cu) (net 31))
 (segment (start 76.2 106.68) (end 76.2 93.98) (width 0.25) (layer B.Cu) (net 31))
 (segment (start 74.93 107.95) (end 76.2 106.68) (width 0.25) (layer B.Cu) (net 31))
 (segment (start 73.66 107.95) (end 74.93 107.95) (width 0.25) (layer B.Cu) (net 31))
 (segment (start 72.39 106.68) (end 73.66 107.95) (width 0.25) (layer B.Cu) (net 31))
 (segment (start 77.47 128.27) (end 77.47 128.62) (width 0.25) (layer B.Cu) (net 36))
 (segment (start 104.14 88.9) (end 85.09 88.9) (width 0.25) (layer B.Cu) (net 37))
 (segment (start 106.68 91.44) (end 104.14 88.9) (width 0.25) (layer B.Cu) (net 37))
 (segment (start 106.68 130.81) (end 106.68 91.44) (width 0.25) (layer B.Cu) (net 37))
 (segment (start 84.74 133.35) (end 104.14 133.35) (width 0.25) (layer B.Cu) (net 37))
 (segment (start 104.14 133.35) (end 106.68 130.81) (width 0.25) (layer B.Cu) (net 37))
 (segment (start 80.01 128.27) (end 80.01 128.62) (width 0.25) (layer B.Cu) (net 37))
 (segment (start 80.01 128.62) (end 84.74 133.35) (width 0.25) (layer B.Cu) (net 37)))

